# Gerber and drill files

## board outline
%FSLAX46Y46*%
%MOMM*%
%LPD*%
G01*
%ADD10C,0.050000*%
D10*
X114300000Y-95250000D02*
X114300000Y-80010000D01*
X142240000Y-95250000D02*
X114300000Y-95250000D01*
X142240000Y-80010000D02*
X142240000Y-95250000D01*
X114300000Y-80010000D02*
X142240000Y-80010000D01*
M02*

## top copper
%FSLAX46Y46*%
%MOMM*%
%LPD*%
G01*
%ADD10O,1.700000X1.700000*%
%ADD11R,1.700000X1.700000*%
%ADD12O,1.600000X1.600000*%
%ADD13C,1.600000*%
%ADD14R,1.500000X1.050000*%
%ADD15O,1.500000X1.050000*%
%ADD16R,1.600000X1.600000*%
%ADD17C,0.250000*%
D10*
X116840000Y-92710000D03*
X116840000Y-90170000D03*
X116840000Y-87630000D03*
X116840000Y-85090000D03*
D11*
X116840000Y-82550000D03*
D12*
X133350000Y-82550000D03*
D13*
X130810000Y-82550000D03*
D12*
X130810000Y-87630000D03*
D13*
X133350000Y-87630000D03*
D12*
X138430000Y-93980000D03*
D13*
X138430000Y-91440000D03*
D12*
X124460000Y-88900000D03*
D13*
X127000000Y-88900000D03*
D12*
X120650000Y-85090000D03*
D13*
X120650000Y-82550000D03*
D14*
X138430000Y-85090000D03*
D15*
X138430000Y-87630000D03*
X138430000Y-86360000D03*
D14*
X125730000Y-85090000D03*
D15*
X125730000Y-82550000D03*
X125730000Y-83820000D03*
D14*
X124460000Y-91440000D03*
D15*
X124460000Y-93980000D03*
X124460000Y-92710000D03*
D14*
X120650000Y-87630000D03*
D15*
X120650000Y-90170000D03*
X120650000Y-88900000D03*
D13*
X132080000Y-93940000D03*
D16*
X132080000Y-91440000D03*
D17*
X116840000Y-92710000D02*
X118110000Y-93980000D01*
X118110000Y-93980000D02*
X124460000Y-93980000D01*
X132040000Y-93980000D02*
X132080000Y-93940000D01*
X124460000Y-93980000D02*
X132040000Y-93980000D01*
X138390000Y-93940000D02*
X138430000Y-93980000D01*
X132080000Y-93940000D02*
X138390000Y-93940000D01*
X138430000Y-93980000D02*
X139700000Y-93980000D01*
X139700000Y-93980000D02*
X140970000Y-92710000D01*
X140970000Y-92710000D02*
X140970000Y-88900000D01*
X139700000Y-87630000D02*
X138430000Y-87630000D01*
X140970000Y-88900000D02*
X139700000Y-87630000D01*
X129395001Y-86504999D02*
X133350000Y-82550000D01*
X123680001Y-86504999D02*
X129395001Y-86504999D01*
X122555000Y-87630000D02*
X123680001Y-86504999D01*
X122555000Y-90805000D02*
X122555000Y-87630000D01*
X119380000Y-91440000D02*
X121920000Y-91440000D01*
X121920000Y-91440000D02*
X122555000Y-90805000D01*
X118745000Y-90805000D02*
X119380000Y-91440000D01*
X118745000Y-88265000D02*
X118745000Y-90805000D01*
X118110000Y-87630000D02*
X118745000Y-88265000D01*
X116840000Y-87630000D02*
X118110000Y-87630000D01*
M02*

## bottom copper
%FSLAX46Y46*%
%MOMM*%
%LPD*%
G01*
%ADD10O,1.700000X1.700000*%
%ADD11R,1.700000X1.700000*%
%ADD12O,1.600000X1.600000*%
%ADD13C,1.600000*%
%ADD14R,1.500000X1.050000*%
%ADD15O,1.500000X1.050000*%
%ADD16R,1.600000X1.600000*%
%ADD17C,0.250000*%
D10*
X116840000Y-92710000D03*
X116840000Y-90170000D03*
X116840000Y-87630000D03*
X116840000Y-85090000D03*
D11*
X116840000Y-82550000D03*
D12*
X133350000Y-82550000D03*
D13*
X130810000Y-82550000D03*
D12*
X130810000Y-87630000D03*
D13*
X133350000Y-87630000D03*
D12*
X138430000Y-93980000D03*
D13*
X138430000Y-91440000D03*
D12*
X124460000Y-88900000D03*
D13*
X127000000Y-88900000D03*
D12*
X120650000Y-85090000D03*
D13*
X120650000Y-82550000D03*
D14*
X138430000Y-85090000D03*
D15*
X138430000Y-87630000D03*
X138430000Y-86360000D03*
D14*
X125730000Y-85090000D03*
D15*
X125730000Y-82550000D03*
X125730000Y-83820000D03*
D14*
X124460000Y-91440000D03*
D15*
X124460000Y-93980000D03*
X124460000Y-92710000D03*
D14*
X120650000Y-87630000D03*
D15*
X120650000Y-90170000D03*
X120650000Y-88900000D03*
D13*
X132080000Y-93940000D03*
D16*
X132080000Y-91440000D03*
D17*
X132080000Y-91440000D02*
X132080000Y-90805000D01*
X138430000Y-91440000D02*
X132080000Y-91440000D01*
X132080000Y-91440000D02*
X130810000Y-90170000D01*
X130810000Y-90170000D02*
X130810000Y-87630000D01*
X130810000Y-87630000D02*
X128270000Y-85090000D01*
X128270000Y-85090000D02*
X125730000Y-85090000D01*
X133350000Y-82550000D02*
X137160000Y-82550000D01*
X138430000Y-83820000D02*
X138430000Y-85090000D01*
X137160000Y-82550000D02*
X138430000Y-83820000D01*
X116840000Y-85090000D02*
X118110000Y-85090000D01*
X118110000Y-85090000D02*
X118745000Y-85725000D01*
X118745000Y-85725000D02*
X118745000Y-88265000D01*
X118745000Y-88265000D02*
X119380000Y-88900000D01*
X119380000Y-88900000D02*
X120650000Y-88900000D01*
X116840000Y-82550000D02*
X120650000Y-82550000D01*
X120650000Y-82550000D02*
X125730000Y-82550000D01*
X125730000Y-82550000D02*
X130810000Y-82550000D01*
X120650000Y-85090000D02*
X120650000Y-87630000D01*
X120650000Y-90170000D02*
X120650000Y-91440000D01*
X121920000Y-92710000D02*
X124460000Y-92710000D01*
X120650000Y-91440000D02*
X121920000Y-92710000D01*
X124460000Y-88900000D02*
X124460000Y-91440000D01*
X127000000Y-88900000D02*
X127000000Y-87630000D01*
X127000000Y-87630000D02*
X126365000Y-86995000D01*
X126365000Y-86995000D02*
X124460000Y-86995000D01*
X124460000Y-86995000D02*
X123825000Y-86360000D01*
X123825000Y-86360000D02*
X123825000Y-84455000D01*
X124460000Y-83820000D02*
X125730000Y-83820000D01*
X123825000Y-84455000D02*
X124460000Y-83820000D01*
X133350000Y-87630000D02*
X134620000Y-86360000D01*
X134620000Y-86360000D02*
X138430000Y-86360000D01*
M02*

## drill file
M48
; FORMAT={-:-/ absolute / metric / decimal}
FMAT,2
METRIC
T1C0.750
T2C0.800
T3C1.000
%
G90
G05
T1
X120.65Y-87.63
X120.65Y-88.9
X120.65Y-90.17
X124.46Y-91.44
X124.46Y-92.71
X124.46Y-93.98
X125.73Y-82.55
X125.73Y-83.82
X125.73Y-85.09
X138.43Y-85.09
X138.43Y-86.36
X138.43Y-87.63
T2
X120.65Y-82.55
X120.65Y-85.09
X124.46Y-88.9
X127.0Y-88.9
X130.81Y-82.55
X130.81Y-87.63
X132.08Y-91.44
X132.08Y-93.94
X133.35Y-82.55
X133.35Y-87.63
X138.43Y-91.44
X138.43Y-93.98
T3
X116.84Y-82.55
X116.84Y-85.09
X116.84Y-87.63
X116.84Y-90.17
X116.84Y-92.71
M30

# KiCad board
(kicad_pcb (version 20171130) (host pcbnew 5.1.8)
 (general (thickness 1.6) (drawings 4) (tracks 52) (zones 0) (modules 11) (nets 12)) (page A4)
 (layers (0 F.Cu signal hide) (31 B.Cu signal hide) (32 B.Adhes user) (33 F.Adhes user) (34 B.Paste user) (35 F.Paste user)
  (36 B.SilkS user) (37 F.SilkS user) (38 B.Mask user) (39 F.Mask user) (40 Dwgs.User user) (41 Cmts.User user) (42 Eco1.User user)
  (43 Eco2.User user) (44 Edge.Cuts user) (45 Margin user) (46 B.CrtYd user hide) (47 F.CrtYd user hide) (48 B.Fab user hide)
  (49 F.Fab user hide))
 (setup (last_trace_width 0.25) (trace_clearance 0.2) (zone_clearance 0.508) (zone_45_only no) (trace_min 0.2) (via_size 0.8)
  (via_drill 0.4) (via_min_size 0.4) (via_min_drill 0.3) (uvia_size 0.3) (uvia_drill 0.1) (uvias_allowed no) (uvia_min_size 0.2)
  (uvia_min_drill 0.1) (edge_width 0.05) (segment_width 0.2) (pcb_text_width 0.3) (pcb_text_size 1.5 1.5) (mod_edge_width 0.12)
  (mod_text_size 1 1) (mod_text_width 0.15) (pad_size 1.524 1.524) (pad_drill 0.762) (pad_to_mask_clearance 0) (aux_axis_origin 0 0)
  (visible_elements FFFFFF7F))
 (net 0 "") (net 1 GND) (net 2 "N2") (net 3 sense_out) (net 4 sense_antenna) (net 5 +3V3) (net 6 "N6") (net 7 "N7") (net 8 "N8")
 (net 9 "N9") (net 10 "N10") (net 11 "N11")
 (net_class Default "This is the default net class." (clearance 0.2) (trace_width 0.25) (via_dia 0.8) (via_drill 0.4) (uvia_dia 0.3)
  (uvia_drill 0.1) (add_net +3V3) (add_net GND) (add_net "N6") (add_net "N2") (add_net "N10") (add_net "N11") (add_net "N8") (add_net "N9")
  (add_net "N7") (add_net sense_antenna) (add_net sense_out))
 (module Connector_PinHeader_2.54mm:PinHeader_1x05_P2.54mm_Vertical (layer B.Cu) (at 116.84 82.55 180)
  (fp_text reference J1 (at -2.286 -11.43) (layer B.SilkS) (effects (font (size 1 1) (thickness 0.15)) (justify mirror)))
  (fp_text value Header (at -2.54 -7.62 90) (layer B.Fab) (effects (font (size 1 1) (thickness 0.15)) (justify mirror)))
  (pad 5 thru_hole oval (at 0 -10.16 180) (size 1.7 1.7) (drill 1) (layers *.Cu *.Mask) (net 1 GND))
  (pad 4 thru_hole oval (at 0 -7.62 180) (size 1.7 1.7) (drill 1) (layers *.Cu *.Mask) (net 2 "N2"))
  (pad 3 thru_hole oval (at 0 -5.08 180) (size 1.7 1.7) (drill 1) (layers *.Cu *.Mask) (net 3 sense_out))
  (pad 2 thru_hole oval (at 0 -2.54 180) (size 1.7 1.7) (drill 1) (layers *.Cu *.Mask) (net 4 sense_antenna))
  (pad 1 thru_hole rect (at 0 0 180) (size 1.7 1.7) (drill 1) (layers *.Cu *.Mask) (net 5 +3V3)))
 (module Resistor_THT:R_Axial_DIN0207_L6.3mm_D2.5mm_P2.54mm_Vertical (layer F.Cu) (at 130.81 82.55)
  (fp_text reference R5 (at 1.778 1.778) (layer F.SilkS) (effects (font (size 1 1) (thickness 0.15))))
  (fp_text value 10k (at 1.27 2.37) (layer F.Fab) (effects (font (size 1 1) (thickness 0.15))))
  (pad 2 thru_hole oval (at 2.54 0) (size 1.6 1.6) (drill 0.8) (layers *.Cu *.Mask) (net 3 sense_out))
  (pad 1 thru_hole circle (at 0 0) (size 1.6 1.6) (drill 0.8) (layers *.Cu *.Mask) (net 5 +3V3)))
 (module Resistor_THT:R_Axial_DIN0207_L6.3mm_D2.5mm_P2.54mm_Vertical (layer F.Cu) (at 133.35 87.63 180)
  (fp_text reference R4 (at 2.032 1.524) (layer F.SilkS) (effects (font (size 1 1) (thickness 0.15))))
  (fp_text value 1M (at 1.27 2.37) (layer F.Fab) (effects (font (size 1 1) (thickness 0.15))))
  (pad 2 thru_hole oval (at 2.54 0 180) (size 1.6 1.6) (drill 0.8) (layers *.Cu *.Mask) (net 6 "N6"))
  (pad 1 thru_hole circle (at 0 0 180) (size 1.6 1.6) (drill 0.8) (layers *.Cu *.Mask) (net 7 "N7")))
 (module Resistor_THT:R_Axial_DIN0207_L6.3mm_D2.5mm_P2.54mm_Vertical (layer F.Cu) (at 138.43 91.44 270)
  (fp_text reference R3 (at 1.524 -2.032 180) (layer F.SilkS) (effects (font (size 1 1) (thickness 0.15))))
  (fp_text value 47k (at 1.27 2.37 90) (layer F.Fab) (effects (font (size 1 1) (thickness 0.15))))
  (pad 2 thru_hole oval (at 2.54 0 270) (size 1.6 1.6) (drill 0.8) (layers *.Cu *.Mask) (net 1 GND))
  (pad 1 thru_hole circle (at 0 0 270) (size 1.6 1.6) (drill 0.8) (layers *.Cu *.Mask) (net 6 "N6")))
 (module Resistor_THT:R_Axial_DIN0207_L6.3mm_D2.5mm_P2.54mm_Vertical (layer F.Cu) (at 127 88.9 180)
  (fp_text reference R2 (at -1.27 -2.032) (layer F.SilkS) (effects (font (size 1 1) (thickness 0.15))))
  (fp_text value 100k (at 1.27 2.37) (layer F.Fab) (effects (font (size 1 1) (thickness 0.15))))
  (pad 2 thru_hole oval (at 2.54 0 180) (size 1.6 1.6) (drill 0.8) (layers *.Cu *.Mask) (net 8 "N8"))
  (pad 1 thru_hole circle (at 0 0 180) (size 1.6 1.6) (drill 0.8) (layers *.Cu *.Mask) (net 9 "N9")))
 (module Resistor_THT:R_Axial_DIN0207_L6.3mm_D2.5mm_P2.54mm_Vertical (layer F.Cu) (at 120.65 82.55 270)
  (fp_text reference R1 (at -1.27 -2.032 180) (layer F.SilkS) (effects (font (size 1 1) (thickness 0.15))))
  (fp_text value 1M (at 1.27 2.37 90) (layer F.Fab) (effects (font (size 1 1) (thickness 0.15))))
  (pad 2 thru_hole oval (at 2.54 0 270) (size 1.6 1.6) (drill 0.8) (layers *.Cu *.Mask) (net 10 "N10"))
  (pad 1 thru_hole circle (at 0 0 270) (size 1.6 1.6) (drill 0.8) (layers *.Cu *.Mask) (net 5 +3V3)))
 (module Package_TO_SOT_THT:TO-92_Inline (layer F.Cu) (at 138.43 85.09 270)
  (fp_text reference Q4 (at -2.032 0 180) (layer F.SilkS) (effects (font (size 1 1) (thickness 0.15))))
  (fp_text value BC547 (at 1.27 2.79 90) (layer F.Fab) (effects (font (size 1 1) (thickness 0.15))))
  (pad 1 thru_hole rect (at 0 0 270) (size 1.05 1.5) (drill 0.75) (layers *.Cu *.Mask) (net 3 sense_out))
  (pad 3 thru_hole oval (at 2.54 0 270) (size 1.05 1.5) (drill 0.75) (layers *.Cu *.Mask) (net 1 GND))
  (pad 2 thru_hole oval (at 1.27 0 270) (size 1.05 1.5) (drill 0.75) (layers *.Cu *.Mask) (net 7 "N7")))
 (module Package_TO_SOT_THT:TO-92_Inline (layer F.Cu) (at 125.73 85.09 90)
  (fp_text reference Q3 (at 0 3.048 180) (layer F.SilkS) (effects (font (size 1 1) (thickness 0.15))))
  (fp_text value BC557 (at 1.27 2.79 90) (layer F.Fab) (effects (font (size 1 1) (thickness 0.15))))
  (pad 1 thru_hole rect (at 0 0 90) (size 1.05 1.5) (drill 0.75) (layers *.Cu *.Mask) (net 6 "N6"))
  (pad 3 thru_hole oval (at 2.54 0 90) (size 1.05 1.5) (drill 0.75) (layers *.Cu *.Mask) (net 5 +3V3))
  (pad 2 thru_hole oval (at 1.27 0 90) (size 1.05 1.5) (drill 0.75) (layers *.Cu *.Mask) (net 9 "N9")))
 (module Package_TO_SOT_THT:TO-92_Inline (layer F.Cu) (at 124.46 91.44 270)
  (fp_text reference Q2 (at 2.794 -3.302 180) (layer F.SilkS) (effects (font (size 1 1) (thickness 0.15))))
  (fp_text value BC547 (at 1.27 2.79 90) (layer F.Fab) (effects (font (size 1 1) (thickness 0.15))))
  (pad 1 thru_hole rect (at 0 0 270) (size 1.05 1.5) (drill 0.75) (layers *.Cu *.Mask) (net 8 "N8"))
  (pad 3 thru_hole oval (at 2.54 0 270) (size 1.05 1.5) (drill 0.75) (layers *.Cu *.Mask) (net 1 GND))
  (pad 2 thru_hole oval (at 1.27 0 270) (size 1.05 1.5) (drill 0.75) (layers *.Cu *.Mask) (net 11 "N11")))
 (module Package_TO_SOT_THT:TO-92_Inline (layer F.Cu) (at 120.65 87.63 270)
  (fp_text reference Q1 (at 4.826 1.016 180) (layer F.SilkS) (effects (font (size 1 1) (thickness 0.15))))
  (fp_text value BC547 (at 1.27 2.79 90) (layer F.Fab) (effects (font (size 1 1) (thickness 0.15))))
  (pad 1 thru_hole rect (at 0 0 270) (size 1.05 1.5) (drill 0.75) (layers *.Cu *.Mask) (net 10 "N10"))
  (pad 3 thru_hole oval (at 2.54 0 270) (size 1.05 1.5) (drill 0.75) (layers *.Cu *.Mask) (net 11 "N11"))
  (pad 2 thru_hole oval (at 1.27 0 270) (size 1.05 1.5) (drill 0.75) (layers *.Cu *.Mask) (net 4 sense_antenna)))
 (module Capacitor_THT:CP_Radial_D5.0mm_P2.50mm (layer F.Cu) (at 132.08 91.44 270)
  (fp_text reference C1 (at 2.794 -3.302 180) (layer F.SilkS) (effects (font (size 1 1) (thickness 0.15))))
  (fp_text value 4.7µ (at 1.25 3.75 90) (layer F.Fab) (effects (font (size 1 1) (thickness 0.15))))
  (pad 2 thru_hole circle (at 2.5 0 270) (size 1.6 1.6) (drill 0.8) (layers *.Cu *.Mask) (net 1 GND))
  (pad 1 thru_hole rect (at 0 0 270) (size 1.6 1.6) (drill 0.8) (layers *.Cu *.Mask) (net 6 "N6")))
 (gr_line (start 114.3 95.25) (end 114.3 80.01) (layer Edge.Cuts) (width 0.05))
 (gr_line (start 142.24 95.25) (end 114.3 95.25) (layer Edge.Cuts) (width 0.05))
 (gr_line (start 142.24 80.01) (end 142.24 95.25) (layer Edge.Cuts) (width 0.05))
 (gr_line (start 114.3 80.01) (end 142.24 80.01) (layer Edge.Cuts) (width 0.05))
 (segment (start 116.84 92.71) (end 118.11 93.98) (width 0.25) (layer F.Cu) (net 1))
 (segment (start 118.11 93.98) (end 124.46 93.98) (width 0.25) (layer F.Cu) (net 1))
 (segment (start 132.04 93.98) (end 132.08 93.94) (width 0.25) (layer F.Cu) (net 1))
 (segment (start 124.46 93.98) (end 132.04 93.98) (width 0.25) (layer F.Cu) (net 1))
 (segment (start 138.39 93.94) (end 138.43 93.98) (width 0.25) (layer F.Cu) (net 1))
 (segment (start 132.08 93.94) (end 138.39 93.94) (width 0.25) (layer F.Cu) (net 1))
 (segment (start 138.43 93.98) (end 139.7 93.98) (width 0.25) (layer F.Cu) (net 1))
 (segment (start 139.7 93.98) (end 140.97 92.71) (width 0.25) (layer F.Cu) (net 1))
 (segment (start 140.97 92.71) (end 140.97 88.9) (width 0.25) (layer F.Cu) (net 1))
 (segment (start 139.7 87.63) (end 138.43 87.63) (width 0.25) (layer F.Cu) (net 1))
 (segment (start 140.97 88.9) (end 139.7 87.63) (width 0.25) (layer F.Cu) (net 1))
 (segment (start 132.08 91.44) (end 132.08 90.805) (width 0.25) (layer B.Cu) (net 6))
 (segment (start 138.43 91.44) (end 132.08 91.44) (width 0.25) (layer B.Cu) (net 6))
 (segment (start 132.08 91.44) (end 130.81 90.17) (width 0.25) (layer B.Cu) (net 6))
 (segment (start 130.81 90.17) (end 130.81 87.63) (width 0.25) (layer B.Cu) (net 6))
 (segment (start 130.81 87.63) (end 128.27 85.09) (width 0.25) (layer B.Cu) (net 6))
 (segment (start 128.27 85.09) (end 125.73 85.09) (width 0.25) (layer B.Cu) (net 6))
 (segment (start 133.35 82.55) (end 137.16 82.55) (width 0.25) (layer B.Cu) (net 3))
 (segment (start 138.43 83.82) (end 138.43 85.09) (width 0.25) (layer B.Cu) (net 3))
 (segment (start 137.16 82.55) (end 138.43 83.82) (width 0.25) (layer B.Cu) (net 3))
 (segment (start 129.395001 86.504999) (end 133.35 82.55) (width 0.25) (layer F.Cu) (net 3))
 (segment (start 123.680001 86.504999) (end 129.395001 86.504999) (width 0.25) (layer F.Cu) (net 3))
 (segment (start 122.555 87.63) (end 123.680001 86.504999) (width 0.25) (layer F.Cu) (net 3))
 (segment (start 122.555 90.805) (end 122.555 87.63) (width 0.25) (layer F.Cu) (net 3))
 (segment (start 119.38 91.44) (end 121.92 91.44) (width 0.25) (layer F.Cu) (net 3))
 (segment (start 121.92 91.44) (end 122.555 90.805) (width 0.25) (layer F.Cu) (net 3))
 (segment (start 118.745 90.805) (end 119.38 91.44) (width 0.25) (layer F.Cu) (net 3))
 (segment (start 118.745 88.265) (end 118.745 90.805) (width 0.25) (layer F.Cu) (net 3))
 (segment (start 118.11 87.63) (end 118.745 88.265) (width 0.25) (layer F.Cu) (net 3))
 (segment (start 116.84 87.63) (end 118.11 87.63) (width 0.25) (layer F.Cu) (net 3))
 (segment (start 116.84 85.09) (end 118.11 85.09) (width 0.25) (layer B.Cu) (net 4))
 (segment (start 118.11 85.09) (end 118.745 85.725) (width 0.25) (layer B.Cu) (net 4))
 (segment (start 118.745 85.725) (end 118.745 88.265) (width 0.25) (layer B.Cu) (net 4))
 (segment (start 118.745 88.265) (end 119.38 88.9) (width 0.25) (layer B.Cu) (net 4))
 (segment (start 119.38 88.9) (end 120.65 88.9) (width 0.25) (layer B.Cu) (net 4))
 (segment (start 116.84 82.55) (end 120.65 82.55) (width 0.25) (layer B.Cu) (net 5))
 (segment (start 120.65 82.55) (end 125.73 82.55) (width 0.25) (layer B.Cu) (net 5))
 (segment (start 125.73 82.55) (end 130.81 82.55) (width 0.25) (layer B.Cu) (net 5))
 (segment (start 120.65 85.09) (end 120.65 87.63) (width 0.25) (layer B.Cu) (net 10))
 (segment (start 120.65 90.17) (end 120.65 91.44) (width 0.25) (layer B.Cu) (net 11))
 (segment (start 121.92 92.71) (end 124.46 92.71) (width 0.25) (layer B.Cu) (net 11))
 (segment (start 120.65 91.44) (end 121.92 92.71) (width 0.25) (layer B.Cu) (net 11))
 (segment (start 124.46 88.9) (end 124.46 91.44) (width 0.25) (layer B.Cu) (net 8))
 (segment (start 127 88.9) (end 127 87.63) (width 0.25) (layer B.Cu) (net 9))
 (segment (start 127 87.63) (end 126.365 86.995) (width 0.25) (layer B.Cu) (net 9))
 (segment (start 126.365 86.995) (end 124.46 86.995) (width 0.25) (layer B.Cu) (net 9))
 (segment (start 124.46 86.995) (end 123.825 86.36) (width 0.25) (layer B.Cu) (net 9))
 (segment (start 123.825 86.36) (end 123.825 84.455) (width 0.25) (layer B.Cu) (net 9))
 (segment (start 124.46 83.82) (end 125.73 83.82) (width 0.25) (layer B.Cu) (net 9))
 (segment (start 123.825 84.455) (end 124.46 83.82) (width 0.25) (layer B.Cu) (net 9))
 (segment (start 133.35 87.63) (end 134.62 86.36) (width 0.25) (layer B.Cu) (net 7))
 (segment (start 134.62 86.36) (end 138.43 86.36) (width 0.25) (layer B.Cu) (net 7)))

